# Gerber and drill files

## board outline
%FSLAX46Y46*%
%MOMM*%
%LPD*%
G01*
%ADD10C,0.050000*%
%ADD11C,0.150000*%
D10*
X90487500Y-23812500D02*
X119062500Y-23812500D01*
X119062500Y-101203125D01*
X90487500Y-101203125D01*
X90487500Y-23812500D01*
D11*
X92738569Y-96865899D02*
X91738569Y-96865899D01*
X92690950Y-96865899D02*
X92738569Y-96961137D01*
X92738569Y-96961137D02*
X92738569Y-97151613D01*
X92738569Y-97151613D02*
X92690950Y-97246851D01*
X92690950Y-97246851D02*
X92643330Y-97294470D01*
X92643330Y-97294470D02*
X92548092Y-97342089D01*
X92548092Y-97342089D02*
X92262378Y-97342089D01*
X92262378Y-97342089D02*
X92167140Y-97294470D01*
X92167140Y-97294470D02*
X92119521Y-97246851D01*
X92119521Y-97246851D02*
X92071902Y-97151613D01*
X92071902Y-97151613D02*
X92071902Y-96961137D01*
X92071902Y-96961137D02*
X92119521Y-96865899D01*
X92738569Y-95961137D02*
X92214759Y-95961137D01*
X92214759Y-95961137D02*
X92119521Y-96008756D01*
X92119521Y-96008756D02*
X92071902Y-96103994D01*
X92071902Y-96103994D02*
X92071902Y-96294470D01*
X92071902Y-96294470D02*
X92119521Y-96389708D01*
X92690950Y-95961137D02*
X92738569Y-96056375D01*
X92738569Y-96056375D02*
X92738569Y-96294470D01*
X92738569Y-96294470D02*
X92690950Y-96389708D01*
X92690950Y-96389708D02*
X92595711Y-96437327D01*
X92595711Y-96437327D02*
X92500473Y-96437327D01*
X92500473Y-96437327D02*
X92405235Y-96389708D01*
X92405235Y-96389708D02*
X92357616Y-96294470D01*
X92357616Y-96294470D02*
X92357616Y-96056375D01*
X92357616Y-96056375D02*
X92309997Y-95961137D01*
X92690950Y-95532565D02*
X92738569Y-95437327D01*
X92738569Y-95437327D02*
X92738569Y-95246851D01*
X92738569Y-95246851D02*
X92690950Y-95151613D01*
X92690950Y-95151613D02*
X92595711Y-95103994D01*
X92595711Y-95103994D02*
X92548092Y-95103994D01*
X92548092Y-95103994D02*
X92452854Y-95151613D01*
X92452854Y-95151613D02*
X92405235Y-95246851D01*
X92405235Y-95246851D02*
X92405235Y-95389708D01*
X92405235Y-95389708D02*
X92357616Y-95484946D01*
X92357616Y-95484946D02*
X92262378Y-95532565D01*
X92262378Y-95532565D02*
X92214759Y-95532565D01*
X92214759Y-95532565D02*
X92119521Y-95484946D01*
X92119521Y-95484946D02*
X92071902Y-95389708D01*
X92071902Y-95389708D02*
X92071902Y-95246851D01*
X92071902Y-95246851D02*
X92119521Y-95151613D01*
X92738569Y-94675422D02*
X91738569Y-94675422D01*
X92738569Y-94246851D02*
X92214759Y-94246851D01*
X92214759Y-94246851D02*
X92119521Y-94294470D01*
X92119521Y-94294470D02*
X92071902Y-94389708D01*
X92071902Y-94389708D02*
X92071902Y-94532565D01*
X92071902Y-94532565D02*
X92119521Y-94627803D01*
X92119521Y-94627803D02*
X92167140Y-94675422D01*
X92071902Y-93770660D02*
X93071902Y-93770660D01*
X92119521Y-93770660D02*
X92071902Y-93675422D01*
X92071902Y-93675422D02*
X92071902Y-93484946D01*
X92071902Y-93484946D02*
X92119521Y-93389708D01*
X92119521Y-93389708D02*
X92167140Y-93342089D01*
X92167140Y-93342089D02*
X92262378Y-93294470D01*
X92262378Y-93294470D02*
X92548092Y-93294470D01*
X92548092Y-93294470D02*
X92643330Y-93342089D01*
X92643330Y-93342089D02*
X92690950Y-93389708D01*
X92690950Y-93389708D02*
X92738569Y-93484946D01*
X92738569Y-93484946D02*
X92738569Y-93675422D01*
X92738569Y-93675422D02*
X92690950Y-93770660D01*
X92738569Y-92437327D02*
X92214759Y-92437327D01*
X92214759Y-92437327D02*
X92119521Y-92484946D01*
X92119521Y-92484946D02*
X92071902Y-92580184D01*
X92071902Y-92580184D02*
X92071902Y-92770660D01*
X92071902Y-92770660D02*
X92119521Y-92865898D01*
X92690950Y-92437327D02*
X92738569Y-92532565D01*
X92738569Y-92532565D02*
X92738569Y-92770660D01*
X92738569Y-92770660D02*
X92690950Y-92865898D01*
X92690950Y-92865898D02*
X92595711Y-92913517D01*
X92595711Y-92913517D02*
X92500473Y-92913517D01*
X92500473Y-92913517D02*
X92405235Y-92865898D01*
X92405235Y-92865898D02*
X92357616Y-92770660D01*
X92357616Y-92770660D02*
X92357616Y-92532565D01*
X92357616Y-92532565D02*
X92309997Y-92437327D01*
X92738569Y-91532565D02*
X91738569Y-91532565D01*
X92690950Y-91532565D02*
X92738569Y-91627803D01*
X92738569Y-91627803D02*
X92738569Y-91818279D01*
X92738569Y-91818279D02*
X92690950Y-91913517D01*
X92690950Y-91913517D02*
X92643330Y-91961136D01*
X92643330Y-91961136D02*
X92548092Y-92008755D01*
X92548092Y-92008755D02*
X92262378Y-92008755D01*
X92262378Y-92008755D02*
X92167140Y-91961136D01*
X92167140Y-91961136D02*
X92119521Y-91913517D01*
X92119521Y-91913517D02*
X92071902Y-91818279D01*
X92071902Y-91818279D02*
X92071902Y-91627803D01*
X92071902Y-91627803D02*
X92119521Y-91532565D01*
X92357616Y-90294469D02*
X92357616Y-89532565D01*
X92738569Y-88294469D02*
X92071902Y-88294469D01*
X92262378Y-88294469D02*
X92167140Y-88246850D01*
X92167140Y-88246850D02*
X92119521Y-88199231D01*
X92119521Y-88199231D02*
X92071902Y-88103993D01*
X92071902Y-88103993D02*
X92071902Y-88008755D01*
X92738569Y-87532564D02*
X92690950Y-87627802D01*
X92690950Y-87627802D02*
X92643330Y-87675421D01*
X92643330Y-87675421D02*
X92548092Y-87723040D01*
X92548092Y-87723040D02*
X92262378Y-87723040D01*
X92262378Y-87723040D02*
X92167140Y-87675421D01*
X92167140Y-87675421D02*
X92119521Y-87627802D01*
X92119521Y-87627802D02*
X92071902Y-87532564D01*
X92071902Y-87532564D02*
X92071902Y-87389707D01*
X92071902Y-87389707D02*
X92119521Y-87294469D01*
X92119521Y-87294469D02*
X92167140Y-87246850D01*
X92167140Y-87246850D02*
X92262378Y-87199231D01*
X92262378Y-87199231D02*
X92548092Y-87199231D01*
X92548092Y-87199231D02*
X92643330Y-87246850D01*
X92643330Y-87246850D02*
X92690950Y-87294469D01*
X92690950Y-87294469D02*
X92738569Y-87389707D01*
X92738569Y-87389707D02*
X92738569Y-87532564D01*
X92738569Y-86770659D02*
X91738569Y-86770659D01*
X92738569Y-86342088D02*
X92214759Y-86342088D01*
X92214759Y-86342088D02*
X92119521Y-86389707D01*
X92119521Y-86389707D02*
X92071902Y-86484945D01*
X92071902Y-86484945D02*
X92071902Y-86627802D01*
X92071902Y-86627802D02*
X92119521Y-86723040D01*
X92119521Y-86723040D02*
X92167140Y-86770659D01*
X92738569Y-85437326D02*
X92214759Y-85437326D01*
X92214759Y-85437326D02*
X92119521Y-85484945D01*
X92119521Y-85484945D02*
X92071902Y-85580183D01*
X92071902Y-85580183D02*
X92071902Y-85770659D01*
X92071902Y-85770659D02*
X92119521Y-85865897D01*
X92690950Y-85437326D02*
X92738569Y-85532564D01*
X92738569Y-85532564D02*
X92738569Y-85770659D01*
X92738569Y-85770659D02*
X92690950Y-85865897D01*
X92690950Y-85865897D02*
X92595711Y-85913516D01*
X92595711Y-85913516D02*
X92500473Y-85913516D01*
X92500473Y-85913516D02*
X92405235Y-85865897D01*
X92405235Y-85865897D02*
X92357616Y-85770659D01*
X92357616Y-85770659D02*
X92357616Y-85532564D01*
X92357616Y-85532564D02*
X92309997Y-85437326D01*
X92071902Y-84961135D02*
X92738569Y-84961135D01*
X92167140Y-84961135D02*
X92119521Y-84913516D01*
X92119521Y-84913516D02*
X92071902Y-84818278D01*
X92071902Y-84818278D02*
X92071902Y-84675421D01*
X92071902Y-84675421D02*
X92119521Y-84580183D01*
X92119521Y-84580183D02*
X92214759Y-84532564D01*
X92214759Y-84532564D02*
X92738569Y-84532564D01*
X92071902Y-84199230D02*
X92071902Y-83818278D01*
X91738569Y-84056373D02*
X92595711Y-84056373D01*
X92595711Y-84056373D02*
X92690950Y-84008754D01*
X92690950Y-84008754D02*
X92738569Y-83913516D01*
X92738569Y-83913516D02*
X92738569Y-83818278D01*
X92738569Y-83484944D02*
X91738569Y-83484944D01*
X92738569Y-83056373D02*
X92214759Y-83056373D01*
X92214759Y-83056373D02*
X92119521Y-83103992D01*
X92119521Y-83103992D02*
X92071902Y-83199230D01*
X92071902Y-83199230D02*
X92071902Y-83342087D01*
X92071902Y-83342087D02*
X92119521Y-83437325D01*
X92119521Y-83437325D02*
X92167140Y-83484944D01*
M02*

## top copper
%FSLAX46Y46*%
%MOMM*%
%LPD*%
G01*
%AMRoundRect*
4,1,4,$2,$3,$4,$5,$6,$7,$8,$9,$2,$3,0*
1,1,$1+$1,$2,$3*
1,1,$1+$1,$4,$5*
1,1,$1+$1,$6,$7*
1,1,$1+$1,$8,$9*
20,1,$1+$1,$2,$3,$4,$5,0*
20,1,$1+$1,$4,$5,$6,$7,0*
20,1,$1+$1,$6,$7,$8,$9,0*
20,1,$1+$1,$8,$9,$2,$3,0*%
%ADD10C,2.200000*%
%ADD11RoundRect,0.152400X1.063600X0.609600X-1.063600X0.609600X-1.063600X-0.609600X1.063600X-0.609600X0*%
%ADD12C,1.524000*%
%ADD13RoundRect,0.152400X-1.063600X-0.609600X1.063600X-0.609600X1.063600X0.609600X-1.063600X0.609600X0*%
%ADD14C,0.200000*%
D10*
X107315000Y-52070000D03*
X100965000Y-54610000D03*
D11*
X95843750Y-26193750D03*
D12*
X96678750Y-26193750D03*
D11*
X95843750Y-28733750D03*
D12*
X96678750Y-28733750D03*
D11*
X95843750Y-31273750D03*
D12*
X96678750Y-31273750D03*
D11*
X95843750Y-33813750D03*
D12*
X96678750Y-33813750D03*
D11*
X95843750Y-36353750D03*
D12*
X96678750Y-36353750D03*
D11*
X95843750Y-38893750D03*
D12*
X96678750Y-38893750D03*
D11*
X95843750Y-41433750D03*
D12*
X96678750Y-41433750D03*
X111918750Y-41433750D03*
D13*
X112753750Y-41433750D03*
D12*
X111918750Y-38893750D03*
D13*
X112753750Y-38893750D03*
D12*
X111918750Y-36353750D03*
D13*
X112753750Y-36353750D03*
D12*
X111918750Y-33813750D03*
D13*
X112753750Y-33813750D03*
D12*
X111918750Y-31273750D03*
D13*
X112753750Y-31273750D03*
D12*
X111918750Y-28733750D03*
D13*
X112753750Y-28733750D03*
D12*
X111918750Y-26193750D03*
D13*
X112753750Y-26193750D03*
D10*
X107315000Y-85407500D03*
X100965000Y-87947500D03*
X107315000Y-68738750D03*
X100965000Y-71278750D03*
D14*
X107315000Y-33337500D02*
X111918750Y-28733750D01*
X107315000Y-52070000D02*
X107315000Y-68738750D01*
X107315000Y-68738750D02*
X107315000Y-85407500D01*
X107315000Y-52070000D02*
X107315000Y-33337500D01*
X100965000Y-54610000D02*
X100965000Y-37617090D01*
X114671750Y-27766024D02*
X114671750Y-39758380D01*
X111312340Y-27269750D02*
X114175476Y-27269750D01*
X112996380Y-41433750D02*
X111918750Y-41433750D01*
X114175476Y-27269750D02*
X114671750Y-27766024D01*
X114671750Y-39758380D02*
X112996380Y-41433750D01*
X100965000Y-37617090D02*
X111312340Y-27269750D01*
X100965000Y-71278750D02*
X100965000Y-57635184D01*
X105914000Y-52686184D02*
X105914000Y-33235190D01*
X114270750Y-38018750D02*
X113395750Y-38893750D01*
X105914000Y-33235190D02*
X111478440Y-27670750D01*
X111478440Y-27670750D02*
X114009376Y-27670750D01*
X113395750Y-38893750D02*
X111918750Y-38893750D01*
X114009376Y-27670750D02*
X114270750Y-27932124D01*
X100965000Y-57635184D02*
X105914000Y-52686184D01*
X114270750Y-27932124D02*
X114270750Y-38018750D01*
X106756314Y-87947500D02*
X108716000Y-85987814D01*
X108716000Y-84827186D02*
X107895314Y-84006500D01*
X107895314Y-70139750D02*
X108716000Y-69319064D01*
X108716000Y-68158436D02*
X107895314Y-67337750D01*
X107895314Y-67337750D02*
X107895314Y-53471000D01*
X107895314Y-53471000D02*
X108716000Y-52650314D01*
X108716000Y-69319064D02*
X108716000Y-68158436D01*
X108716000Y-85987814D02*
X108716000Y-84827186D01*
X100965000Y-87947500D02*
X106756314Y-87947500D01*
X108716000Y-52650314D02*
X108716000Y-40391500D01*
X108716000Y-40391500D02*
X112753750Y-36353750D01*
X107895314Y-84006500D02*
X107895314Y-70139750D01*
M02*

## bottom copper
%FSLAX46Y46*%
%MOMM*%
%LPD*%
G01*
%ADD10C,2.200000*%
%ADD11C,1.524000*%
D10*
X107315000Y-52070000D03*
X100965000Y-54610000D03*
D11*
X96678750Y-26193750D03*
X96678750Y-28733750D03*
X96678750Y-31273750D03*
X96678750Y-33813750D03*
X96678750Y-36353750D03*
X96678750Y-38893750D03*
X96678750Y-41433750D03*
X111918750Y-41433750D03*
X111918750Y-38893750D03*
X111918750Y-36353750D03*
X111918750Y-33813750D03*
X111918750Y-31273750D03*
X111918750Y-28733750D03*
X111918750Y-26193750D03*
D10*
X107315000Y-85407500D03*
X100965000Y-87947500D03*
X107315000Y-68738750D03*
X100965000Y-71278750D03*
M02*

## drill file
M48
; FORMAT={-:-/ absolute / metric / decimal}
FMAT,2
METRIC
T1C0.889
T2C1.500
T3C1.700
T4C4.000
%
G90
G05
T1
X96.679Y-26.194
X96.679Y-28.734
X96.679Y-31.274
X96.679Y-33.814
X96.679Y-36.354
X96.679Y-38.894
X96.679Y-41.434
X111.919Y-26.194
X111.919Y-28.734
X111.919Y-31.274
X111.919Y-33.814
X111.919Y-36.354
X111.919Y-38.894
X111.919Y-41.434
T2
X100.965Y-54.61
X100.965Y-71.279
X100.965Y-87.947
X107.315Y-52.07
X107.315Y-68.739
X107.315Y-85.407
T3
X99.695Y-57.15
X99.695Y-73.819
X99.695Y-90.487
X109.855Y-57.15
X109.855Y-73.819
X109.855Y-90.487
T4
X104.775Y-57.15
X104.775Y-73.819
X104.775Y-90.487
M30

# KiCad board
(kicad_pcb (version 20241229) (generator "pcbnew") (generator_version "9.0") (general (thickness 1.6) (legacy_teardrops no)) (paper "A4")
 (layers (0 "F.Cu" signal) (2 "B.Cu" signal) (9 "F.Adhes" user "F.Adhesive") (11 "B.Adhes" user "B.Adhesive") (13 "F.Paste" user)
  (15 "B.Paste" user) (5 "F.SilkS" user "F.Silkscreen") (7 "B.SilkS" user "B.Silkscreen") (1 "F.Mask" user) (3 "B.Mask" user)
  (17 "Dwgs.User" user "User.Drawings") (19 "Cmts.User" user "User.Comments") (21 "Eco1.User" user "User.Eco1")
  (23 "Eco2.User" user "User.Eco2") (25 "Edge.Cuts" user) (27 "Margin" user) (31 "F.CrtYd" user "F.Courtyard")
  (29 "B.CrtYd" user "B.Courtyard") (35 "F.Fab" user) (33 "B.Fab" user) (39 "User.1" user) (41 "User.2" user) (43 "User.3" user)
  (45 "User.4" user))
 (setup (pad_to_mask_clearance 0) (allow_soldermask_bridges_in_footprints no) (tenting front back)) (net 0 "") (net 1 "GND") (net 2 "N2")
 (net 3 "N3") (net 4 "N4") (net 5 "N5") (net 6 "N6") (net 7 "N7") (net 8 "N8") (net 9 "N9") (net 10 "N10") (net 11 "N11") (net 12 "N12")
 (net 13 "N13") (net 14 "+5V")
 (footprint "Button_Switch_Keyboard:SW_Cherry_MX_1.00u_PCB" (layer "F.Cu") (at 107.315 52.07)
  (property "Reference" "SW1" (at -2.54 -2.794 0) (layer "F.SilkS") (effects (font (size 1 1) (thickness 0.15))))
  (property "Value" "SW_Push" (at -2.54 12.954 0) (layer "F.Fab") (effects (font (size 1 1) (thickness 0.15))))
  (pad "" np_thru_hole circle (at -7.62 5.08) (size 1.7 1.7) (drill 1.7) (layers "*.Cu" "*.Mask"))
  (pad "" np_thru_hole circle (at -2.54 5.08) (size 4 4) (drill 4) (layers "*.Cu" "*.Mask"))
  (pad "" np_thru_hole circle (at 2.54 5.08) (size 1.7 1.7) (drill 1.7) (layers "*.Cu" "*.Mask"))
  (pad "1" thru_hole circle (at 0 0) (size 2.2 2.2) (drill 1.5) (layers "*.Cu" "*.Mask") (remove_unused_layers no) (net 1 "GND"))
  (pad "2" thru_hole circle (at -6.35 2.54) (size 2.2 2.2) (drill 1.5) (layers "*.Cu" "*.Mask") (remove_unused_layers no) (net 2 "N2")))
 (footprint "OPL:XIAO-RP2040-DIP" (layer "F.Cu") (at 104.29875 33.81375)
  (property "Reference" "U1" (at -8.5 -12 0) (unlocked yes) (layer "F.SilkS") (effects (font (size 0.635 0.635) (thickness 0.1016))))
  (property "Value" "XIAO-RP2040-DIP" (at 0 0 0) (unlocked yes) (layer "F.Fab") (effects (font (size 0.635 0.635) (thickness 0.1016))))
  (pad "1" smd roundrect (at -8.455 -7.62 180) (size 2.432 1.524) (layers "F.Cu" "F.Mask") (roundrect_rratio 0.1) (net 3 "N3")
   (thermal_bridge_angle 45))
  (pad "1" thru_hole circle (at -7.62 -7.62 180) (size 1.524 1.524) (drill 0.889) (layers "*.Cu" "*.Mask") (remove_unused_layers no)
   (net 3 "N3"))
  (pad "2" smd roundrect (at -8.455 -5.08 180) (size 2.432 1.524) (layers "F.Cu" "F.Mask") (roundrect_rratio 0.1) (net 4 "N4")
   (thermal_bridge_angle 45))
  (pad "2" thru_hole circle (at -7.62 -5.08 180) (size 1.524 1.524) (drill 0.889) (layers "*.Cu" "*.Mask") (remove_unused_layers no)
   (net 4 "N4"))
  (pad "3" smd roundrect (at -8.455 -2.54 180) (size 2.432 1.524) (layers "F.Cu" "F.Mask") (roundrect_rratio 0.1) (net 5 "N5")
   (thermal_bridge_angle 45))
  (pad "3" thru_hole circle (at -7.62 -2.54 180) (size 1.524 1.524) (drill 0.889) (layers "*.Cu" "*.Mask") (remove_unused_layers no)
   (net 5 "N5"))
  (pad "4" smd roundrect (at -8.455 0 180) (size 2.432 1.524) (layers "F.Cu" "F.Mask") (roundrect_rratio 0.1) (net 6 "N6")
   (thermal_bridge_angle 45))
  (pad "4" thru_hole circle (at -7.62 0 180) (size 1.524 1.524) (drill 0.889) (layers "*.Cu" "*.Mask") (remove_unused_layers no)
   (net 6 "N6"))
  (pad "5" smd roundrect (at -8.455 2.54 180) (size 2.432 1.524) (layers "F.Cu" "F.Mask") (roundrect_rratio 0.1) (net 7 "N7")
   (thermal_bridge_angle 45))
  (pad "5" thru_hole circle (at -7.62 2.54 180) (size 1.524 1.524) (drill 0.889) (layers "*.Cu" "*.Mask") (remove_unused_layers no)
   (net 7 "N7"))
  (pad "6" smd roundrect (at -8.455 5.08 180) (size 2.432 1.524) (layers "F.Cu" "F.Mask") (roundrect_rratio 0.1) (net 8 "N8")
   (thermal_bridge_angle 45))
  (pad "6" thru_hole circle (at -7.62 5.08 180) (size 1.524 1.524) (drill 0.889) (layers "*.Cu" "*.Mask") (remove_unused_layers no)
   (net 8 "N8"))
  (pad "7" smd roundrect (at -8.455 7.62 180) (size 2.432 1.524) (layers "F.Cu" "F.Mask") (roundrect_rratio 0.1) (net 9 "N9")
   (thermal_bridge_angle 45))
  (pad "7" thru_hole circle (at -7.62 7.62 180) (size 1.524 1.524) (drill 0.889) (layers "*.Cu" "*.Mask") (remove_unused_layers no)
   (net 9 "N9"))
  (pad "8" thru_hole circle (at 7.62 7.62) (size 1.524 1.524) (drill 0.889) (layers "*.Cu" "*.Mask") (remove_unused_layers no) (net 2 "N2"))
  (pad "8" smd roundrect (at 8.455 7.62) (size 2.432 1.524) (layers "F.Cu" "F.Mask") (roundrect_rratio 0.1) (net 2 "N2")
   (thermal_bridge_angle 45))
  (pad "9" thru_hole circle (at 7.62 5.08) (size 1.524 1.524) (drill 0.889) (layers "*.Cu" "*.Mask") (remove_unused_layers no)
   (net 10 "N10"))
  (pad "9" smd roundrect (at 8.455 5.08) (size 2.432 1.524) (layers "F.Cu" "F.Mask") (roundrect_rratio 0.1) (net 10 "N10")
   (thermal_bridge_angle 45))
  (pad "10" thru_hole circle (at 7.62 2.54) (size 1.524 1.524) (drill 0.889) (layers "*.Cu" "*.Mask") (remove_unused_layers no)
   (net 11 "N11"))
  (pad "10" smd roundrect (at 8.455 2.54) (size 2.432 1.524) (layers "F.Cu" "F.Mask") (roundrect_rratio 0.1) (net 11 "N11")
   (thermal_bridge_angle 45))
  (pad "11" thru_hole circle (at 7.62 0) (size 1.524 1.524) (drill 0.889) (layers "*.Cu" "*.Mask") (remove_unused_layers no) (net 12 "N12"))
  (pad "11" smd roundrect (at 8.455 0) (size 2.432 1.524) (layers "F.Cu" "F.Mask") (roundrect_rratio 0.1) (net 12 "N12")
   (thermal_bridge_angle 45))
  (pad "12" thru_hole circle (at 7.62 -2.54) (size 1.524 1.524) (drill 0.889) (layers "*.Cu" "*.Mask") (remove_unused_layers no)
   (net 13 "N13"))
  (pad "12" smd roundrect (at 8.455 -2.54) (size 2.432 1.524) (layers "F.Cu" "F.Mask") (roundrect_rratio 0.1) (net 13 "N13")
   (thermal_bridge_angle 45))
  (pad "13" thru_hole circle (at 7.62 -5.08) (size 1.524 1.524) (drill 0.889) (layers "*.Cu" "*.Mask") (remove_unused_layers no)
   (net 1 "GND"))
  (pad "13" smd roundrect (at 8.455 -5.08) (size 2.432 1.524) (layers "F.Cu" "F.Mask") (roundrect_rratio 0.1) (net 1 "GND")
   (thermal_bridge_angle 45))
  (pad "14" thru_hole circle (at 7.62 -7.62) (size 1.524 1.524) (drill 0.889) (layers "*.Cu" "*.Mask") (remove_unused_layers no)
   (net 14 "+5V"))
  (pad "14" smd roundrect (at 8.455 -7.62) (size 2.432 1.524) (layers "F.Cu" "F.Mask") (roundrect_rratio 0.1) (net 14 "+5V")
   (thermal_bridge_angle 45)))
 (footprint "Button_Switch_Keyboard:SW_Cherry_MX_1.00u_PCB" (layer "F.Cu") (at 107.315 85.4075)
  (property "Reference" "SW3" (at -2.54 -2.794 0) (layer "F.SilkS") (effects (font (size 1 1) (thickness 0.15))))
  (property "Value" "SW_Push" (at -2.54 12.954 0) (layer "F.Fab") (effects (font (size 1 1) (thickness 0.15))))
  (pad "" np_thru_hole circle (at -7.62 5.08) (size 1.7 1.7) (drill 1.7) (layers "*.Cu" "*.Mask"))
  (pad "" np_thru_hole circle (at -2.54 5.08) (size 4 4) (drill 4) (layers "*.Cu" "*.Mask"))
  (pad "" np_thru_hole circle (at 2.54 5.08) (size 1.7 1.7) (drill 1.7) (layers "*.Cu" "*.Mask"))
  (pad "1" thru_hole circle (at 0 0) (size 2.2 2.2) (drill 1.5) (layers "*.Cu" "*.Mask") (remove_unused_layers no) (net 1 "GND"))
  (pad "2" thru_hole circle (at -6.35 2.54) (size 2.2 2.2) (drill 1.5) (layers "*.Cu" "*.Mask") (remove_unused_layers no) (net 11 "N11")))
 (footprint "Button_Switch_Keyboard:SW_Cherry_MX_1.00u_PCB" (layer "F.Cu") (at 107.315 68.73875)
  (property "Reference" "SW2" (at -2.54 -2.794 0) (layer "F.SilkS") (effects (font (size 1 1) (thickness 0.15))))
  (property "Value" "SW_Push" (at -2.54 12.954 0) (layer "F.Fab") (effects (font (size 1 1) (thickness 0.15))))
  (pad "" np_thru_hole circle (at -7.62 5.08) (size 1.7 1.7) (drill 1.7) (layers "*.Cu" "*.Mask"))
  (pad "" np_thru_hole circle (at -2.54 5.08) (size 4 4) (drill 4) (layers "*.Cu" "*.Mask"))
  (pad "" np_thru_hole circle (at 2.54 5.08) (size 1.7 1.7) (drill 1.7) (layers "*.Cu" "*.Mask"))
  (pad "1" thru_hole circle (at 0 0) (size 2.2 2.2) (drill 1.5) (layers "*.Cu" "*.Mask") (remove_unused_layers no) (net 1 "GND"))
  (pad "2" thru_hole circle (at -6.35 2.54) (size 2.2 2.2) (drill 1.5) (layers "*.Cu" "*.Mask") (remove_unused_layers no) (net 10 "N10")))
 (gr_rect (start 90.4875 23.8125) (end 119.0625 101.203125) (stroke (width 0.05) (type default)) (fill no) (layer "Edge.Cuts"))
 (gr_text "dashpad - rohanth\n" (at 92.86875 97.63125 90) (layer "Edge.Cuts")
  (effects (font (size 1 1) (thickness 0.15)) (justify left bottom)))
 (segment (start 107.315 33.3375) (end 111.91875 28.73375) (width 0.2) (layer "F.Cu") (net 1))
 (segment (start 107.315 52.07) (end 107.315 68.73875) (width 0.2) (layer "F.Cu") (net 1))
 (segment (start 107.315 68.73875) (end 107.315 85.4075) (width 0.2) (layer "F.Cu") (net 1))
 (segment (start 107.315 52.07) (end 107.315 33.3375) (width 0.2) (layer "F.Cu") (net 1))
 (segment (start 100.965 54.61) (end 100.965 37.61709) (width 0.2) (layer "F.Cu") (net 2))
 (segment (start 114.67175 27.766024) (end 114.67175 39.75838) (width 0.2) (layer "F.Cu") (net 2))
 (segment (start 111.31234 27.26975) (end 114.175476 27.26975) (width 0.2) (layer "F.Cu") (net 2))
 (segment (start 112.99638 41.43375) (end 111.91875 41.43375) (width 0.2) (layer "F.Cu") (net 2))
 (segment (start 114.175476 27.26975) (end 114.67175 27.766024) (width 0.2) (layer "F.Cu") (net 2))
 (segment (start 114.67175 39.75838) (end 112.99638 41.43375) (width 0.2) (layer "F.Cu") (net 2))
 (segment (start 100.965 37.61709) (end 111.31234 27.26975) (width 0.2) (layer "F.Cu") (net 2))
 (segment (start 100.965 71.27875) (end 100.965 57.635184) (width 0.2) (layer "F.Cu") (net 10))
 (segment (start 105.914 52.686184) (end 105.914 33.23519) (width 0.2) (layer "F.Cu") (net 10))
 (segment (start 114.27075 38.01875) (end 113.39575 38.89375) (width 0.2) (layer "F.Cu") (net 10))
 (segment (start 105.914 33.23519) (end 111.47844 27.67075) (width 0.2) (layer "F.Cu") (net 10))
 (segment (start 111.47844 27.67075) (end 114.009376 27.67075) (width 0.2) (layer "F.Cu") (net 10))
 (segment (start 113.39575 38.89375) (end 111.91875 38.89375) (width 0.2) (layer "F.Cu") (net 10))
 (segment (start 114.009376 27.67075) (end 114.27075 27.932124) (width 0.2) (layer "F.Cu") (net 10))
 (segment (start 100.965 57.635184) (end 105.914 52.686184) (width 0.2) (layer "F.Cu") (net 10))
 (segment (start 114.27075 27.932124) (end 114.27075 38.01875) (width 0.2) (layer "F.Cu") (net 10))
 (segment (start 106.756314 87.9475) (end 108.716 85.987814) (width 0.2) (layer "F.Cu") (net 11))
 (segment (start 108.716 84.827186) (end 107.895314 84.0065) (width 0.2) (layer "F.Cu") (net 11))
 (segment (start 107.895314 70.13975) (end 108.716 69.319064) (width 0.2) (layer "F.Cu") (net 11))
 (segment (start 108.716 68.158436) (end 107.895314 67.33775) (width 0.2) (layer "F.Cu") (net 11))
 (segment (start 107.895314 67.33775) (end 107.895314 53.471) (width 0.2) (layer "F.Cu") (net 11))
 (segment (start 107.895314 53.471) (end 108.716 52.650314) (width 0.2) (layer "F.Cu") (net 11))
 (segment (start 108.716 69.319064) (end 108.716 68.158436) (width 0.2) (layer "F.Cu") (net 11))
 (segment (start 108.716 85.987814) (end 108.716 84.827186) (width 0.2) (layer "F.Cu") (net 11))
 (segment (start 100.965 87.9475) (end 106.756314 87.9475) (width 0.2) (layer "F.Cu") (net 11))
 (segment (start 108.716 52.650314) (end 108.716 40.3915) (width 0.2) (layer "F.Cu") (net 11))
 (segment (start 108.716 40.3915) (end 112.75375 36.35375) (width 0.2) (layer "F.Cu") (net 11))
 (segment (start 107.895314 84.0065) (end 107.895314 70.13975) (width 0.2) (layer "F.Cu") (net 11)))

